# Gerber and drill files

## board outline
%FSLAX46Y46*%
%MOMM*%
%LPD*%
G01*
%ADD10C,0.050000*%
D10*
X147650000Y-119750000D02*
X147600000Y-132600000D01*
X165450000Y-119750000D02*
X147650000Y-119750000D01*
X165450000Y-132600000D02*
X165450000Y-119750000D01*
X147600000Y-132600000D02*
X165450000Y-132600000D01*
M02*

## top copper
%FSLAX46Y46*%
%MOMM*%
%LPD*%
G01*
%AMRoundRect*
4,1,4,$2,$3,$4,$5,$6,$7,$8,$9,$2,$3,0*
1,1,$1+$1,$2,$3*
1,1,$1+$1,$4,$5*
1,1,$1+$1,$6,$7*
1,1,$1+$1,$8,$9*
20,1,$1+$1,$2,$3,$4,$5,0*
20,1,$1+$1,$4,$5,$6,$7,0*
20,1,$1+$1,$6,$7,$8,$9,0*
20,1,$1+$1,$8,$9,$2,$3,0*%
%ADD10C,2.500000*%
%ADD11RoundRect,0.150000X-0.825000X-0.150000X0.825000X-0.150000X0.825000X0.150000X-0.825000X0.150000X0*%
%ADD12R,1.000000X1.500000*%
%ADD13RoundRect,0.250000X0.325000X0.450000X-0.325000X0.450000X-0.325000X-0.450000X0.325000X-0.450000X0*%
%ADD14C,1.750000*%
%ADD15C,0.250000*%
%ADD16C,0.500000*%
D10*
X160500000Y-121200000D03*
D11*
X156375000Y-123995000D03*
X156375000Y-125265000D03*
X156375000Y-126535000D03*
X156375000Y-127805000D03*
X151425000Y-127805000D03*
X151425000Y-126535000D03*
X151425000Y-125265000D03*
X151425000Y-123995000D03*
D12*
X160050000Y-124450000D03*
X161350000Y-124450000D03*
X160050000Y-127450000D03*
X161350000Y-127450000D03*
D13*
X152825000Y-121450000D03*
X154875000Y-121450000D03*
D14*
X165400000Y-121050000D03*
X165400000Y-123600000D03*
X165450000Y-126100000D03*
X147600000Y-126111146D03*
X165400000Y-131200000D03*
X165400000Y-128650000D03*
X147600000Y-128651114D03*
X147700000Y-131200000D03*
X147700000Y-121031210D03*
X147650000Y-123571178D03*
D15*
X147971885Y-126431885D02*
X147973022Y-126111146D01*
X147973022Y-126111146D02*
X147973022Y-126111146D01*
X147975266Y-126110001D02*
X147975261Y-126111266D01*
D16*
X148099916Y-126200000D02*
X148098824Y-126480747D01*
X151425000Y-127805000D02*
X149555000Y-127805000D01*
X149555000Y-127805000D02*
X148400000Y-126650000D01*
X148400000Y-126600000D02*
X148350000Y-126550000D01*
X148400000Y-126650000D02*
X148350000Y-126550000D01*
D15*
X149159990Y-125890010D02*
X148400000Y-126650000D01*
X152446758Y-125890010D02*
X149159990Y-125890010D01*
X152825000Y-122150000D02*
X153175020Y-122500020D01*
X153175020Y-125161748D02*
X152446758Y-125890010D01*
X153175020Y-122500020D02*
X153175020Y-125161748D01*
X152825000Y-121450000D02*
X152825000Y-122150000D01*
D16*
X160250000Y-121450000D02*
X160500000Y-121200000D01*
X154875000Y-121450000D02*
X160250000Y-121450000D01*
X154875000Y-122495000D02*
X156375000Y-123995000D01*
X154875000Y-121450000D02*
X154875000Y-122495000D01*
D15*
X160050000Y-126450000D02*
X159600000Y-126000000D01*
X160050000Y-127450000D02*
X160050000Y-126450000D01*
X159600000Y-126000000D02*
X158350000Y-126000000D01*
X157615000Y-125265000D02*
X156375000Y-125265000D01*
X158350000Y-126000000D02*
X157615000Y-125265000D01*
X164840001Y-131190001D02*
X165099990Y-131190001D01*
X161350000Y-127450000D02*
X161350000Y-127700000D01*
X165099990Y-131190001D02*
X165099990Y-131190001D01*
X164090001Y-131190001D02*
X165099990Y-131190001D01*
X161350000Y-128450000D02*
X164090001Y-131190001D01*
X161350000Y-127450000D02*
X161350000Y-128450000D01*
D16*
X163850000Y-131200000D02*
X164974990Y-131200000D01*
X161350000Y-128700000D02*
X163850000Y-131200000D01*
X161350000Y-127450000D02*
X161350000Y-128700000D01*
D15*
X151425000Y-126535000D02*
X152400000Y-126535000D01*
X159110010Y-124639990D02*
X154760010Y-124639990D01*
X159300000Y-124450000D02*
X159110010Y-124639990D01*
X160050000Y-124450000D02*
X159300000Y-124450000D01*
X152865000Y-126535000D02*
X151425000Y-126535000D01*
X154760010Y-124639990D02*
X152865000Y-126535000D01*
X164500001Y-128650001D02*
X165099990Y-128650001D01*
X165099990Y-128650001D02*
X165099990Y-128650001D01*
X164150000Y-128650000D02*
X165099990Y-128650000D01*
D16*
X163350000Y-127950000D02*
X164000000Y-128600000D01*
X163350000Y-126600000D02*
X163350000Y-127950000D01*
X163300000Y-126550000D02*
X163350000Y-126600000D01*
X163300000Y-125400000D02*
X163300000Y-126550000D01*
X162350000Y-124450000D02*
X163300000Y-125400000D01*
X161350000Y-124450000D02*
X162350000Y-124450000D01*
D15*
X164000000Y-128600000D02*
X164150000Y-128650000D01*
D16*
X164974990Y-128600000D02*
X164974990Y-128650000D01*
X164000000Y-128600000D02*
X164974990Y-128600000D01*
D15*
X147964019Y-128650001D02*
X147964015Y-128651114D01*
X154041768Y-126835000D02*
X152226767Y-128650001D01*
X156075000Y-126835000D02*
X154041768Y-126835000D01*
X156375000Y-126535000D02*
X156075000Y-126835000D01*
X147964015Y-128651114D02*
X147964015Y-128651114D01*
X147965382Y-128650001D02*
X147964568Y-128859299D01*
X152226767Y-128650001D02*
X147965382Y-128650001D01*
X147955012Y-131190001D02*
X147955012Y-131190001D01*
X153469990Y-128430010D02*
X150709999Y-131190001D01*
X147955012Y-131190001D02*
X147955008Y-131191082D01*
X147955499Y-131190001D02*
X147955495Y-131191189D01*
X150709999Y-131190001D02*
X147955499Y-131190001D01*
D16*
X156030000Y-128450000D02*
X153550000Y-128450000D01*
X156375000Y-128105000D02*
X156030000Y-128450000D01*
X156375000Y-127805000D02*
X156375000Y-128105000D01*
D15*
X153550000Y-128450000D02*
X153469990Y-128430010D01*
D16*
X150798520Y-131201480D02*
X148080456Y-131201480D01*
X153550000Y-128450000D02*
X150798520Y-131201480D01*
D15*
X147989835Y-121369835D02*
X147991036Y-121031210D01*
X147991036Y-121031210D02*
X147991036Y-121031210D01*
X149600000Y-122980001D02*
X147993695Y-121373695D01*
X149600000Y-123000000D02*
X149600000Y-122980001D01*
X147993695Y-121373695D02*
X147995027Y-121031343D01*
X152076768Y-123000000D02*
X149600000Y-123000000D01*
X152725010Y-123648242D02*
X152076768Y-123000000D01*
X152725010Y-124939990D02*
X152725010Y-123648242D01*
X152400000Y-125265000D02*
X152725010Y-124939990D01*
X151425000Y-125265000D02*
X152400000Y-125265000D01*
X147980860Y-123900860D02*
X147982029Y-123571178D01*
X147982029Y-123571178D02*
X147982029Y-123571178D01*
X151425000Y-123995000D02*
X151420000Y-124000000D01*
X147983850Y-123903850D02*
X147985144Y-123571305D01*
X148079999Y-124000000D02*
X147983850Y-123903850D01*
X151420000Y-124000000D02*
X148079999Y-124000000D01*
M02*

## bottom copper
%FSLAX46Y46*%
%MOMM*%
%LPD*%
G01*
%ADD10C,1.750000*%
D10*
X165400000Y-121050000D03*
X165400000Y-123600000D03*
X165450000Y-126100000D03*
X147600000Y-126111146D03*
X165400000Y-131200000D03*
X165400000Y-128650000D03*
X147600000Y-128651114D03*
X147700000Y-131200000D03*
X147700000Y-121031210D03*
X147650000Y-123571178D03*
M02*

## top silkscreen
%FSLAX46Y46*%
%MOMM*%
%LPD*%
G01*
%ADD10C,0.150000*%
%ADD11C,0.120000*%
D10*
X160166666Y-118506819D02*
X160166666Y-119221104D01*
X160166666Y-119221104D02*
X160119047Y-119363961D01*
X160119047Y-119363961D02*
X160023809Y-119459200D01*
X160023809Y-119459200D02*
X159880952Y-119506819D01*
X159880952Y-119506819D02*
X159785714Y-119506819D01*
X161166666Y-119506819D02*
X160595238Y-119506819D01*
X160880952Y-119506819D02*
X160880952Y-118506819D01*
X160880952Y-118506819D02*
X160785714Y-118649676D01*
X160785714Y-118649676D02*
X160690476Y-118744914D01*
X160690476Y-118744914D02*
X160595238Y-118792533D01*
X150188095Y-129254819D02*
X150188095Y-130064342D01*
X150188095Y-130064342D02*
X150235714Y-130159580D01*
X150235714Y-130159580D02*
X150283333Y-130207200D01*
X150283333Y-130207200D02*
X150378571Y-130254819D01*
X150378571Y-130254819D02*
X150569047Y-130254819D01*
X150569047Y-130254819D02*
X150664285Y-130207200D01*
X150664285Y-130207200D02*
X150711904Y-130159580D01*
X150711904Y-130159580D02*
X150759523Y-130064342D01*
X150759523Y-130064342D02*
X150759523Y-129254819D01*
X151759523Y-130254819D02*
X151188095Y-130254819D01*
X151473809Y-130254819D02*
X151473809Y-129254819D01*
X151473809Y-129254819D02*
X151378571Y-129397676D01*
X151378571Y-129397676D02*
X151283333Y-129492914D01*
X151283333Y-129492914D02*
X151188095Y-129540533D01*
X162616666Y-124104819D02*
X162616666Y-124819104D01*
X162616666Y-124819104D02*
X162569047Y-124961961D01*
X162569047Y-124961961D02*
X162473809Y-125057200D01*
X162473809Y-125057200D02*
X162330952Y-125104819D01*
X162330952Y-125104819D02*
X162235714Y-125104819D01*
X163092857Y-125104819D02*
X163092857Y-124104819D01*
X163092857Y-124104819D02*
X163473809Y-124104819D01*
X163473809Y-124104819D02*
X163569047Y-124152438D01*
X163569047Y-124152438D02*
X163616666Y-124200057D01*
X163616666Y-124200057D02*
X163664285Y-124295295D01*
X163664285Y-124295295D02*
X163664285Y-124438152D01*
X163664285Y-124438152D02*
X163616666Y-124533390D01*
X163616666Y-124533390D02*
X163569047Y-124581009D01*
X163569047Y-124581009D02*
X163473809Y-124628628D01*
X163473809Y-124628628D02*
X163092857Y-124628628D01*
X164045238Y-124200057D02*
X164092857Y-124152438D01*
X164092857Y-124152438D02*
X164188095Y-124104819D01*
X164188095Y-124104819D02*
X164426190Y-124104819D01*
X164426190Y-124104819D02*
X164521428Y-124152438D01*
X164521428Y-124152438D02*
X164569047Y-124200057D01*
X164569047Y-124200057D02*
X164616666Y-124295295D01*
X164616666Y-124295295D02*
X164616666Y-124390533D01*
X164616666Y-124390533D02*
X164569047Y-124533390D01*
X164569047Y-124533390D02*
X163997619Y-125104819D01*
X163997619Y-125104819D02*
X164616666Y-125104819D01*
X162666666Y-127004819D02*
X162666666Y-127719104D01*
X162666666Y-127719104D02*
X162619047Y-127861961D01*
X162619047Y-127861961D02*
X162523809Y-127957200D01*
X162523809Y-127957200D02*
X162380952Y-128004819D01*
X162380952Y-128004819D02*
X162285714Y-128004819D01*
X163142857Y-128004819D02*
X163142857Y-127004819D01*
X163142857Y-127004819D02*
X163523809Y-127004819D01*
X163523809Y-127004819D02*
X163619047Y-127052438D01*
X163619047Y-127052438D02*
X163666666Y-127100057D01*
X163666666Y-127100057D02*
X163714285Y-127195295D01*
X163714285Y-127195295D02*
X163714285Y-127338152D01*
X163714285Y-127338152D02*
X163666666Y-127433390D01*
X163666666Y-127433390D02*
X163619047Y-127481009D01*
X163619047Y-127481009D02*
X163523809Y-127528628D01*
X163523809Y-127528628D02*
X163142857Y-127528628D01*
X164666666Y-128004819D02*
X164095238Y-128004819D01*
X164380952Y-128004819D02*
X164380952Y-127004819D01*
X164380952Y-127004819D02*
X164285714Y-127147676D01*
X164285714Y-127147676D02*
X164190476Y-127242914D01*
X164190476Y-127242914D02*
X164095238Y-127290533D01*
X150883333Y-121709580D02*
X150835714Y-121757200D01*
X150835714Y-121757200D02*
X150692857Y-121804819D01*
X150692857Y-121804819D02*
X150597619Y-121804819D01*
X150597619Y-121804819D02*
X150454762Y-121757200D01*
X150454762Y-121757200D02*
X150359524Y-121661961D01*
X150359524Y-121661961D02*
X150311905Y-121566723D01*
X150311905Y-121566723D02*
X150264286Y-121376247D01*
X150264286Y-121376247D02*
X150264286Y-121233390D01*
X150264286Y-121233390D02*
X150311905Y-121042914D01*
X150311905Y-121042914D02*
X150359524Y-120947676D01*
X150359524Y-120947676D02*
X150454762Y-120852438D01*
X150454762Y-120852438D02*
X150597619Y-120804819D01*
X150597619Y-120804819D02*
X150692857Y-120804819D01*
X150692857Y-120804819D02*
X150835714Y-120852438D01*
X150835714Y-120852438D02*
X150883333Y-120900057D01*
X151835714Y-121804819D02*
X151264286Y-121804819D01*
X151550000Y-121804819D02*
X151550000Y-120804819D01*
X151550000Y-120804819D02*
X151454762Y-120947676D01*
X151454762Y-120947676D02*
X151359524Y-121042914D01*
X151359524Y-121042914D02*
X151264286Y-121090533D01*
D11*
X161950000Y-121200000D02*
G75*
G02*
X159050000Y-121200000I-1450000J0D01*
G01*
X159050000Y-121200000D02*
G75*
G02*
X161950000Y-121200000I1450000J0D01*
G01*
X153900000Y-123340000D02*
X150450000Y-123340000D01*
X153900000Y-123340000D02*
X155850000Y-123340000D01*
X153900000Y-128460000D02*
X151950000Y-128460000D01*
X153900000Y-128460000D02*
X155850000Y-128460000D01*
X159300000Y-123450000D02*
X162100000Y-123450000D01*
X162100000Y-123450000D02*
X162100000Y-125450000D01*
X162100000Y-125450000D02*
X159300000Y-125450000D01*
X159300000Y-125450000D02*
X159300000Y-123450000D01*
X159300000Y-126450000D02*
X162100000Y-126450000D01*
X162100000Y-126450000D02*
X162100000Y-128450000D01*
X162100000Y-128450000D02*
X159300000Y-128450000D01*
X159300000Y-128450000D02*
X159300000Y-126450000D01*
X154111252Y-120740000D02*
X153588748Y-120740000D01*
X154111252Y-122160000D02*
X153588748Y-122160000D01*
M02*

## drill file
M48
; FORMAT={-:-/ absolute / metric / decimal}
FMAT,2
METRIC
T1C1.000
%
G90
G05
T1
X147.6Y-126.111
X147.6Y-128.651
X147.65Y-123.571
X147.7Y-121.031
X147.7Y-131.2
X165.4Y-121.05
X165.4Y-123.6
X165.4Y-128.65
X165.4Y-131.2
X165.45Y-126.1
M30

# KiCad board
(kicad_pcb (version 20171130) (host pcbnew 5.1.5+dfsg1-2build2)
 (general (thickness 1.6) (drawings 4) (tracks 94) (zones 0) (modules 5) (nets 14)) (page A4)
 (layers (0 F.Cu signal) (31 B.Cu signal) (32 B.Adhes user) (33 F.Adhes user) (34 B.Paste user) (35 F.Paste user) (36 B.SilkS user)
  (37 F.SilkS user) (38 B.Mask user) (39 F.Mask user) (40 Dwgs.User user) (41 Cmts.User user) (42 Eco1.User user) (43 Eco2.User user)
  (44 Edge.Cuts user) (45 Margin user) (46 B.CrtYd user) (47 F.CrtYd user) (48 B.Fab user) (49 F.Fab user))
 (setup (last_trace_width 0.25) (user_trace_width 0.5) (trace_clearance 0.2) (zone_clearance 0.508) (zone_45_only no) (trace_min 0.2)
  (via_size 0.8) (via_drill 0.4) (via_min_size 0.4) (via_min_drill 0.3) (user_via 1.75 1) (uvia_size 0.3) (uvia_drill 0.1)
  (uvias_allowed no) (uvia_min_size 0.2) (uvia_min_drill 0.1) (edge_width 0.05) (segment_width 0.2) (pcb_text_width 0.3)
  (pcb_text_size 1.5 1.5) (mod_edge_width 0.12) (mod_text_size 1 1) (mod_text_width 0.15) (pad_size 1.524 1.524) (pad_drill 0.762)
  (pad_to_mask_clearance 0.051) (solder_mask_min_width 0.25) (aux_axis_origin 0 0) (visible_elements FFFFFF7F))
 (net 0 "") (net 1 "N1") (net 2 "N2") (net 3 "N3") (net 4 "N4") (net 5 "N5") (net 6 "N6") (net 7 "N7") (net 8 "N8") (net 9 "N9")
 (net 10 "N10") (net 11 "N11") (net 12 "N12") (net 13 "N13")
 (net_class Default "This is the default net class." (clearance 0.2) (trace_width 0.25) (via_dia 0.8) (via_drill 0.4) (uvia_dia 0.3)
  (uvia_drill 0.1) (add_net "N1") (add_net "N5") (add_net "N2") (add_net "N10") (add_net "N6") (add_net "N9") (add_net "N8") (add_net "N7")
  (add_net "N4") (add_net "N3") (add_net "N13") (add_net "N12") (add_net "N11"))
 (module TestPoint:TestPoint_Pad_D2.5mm (layer F.Cu) (at 160.5 121.2)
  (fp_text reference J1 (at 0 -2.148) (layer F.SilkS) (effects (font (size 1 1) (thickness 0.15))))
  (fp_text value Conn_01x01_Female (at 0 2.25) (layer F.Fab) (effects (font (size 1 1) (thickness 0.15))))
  (fp_circle (center 0 0) (end 0 1.45) (layer F.SilkS) (width 0.12))
  (pad 1 smd circle (at 0 0) (size 2.5 2.5) (layers F.Cu F.Mask) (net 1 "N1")))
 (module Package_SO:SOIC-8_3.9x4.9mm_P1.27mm (layer F.Cu) (at 153.9 125.9)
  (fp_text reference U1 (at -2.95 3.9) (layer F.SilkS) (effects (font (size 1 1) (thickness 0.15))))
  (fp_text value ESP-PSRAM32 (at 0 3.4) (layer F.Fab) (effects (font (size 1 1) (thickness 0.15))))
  (fp_line (start 0 -2.56) (end -3.45 -2.56) (layer F.SilkS) (width 0.12))
  (fp_line (start 0 -2.56) (end 1.95 -2.56) (layer F.SilkS) (width 0.12))
  (fp_line (start 0 2.56) (end -1.95 2.56) (layer F.SilkS) (width 0.12))
  (fp_line (start 0 2.56) (end 1.95 2.56) (layer F.SilkS) (width 0.12))
  (pad 8 smd roundrect (at 2.475 -1.905) (size 1.95 0.6) (layers F.Cu F.Paste F.Mask) (roundrect_rratio 0.25) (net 1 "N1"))
  (pad 7 smd roundrect (at 2.475 -0.635) (size 1.95 0.6) (layers F.Cu F.Paste F.Mask) (roundrect_rratio 0.25) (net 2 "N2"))
  (pad 6 smd roundrect (at 2.475 0.635) (size 1.95 0.6) (layers F.Cu F.Paste F.Mask) (roundrect_rratio 0.25) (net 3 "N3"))
  (pad 5 smd roundrect (at 2.475 1.905) (size 1.95 0.6) (layers F.Cu F.Paste F.Mask) (roundrect_rratio 0.25) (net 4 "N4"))
  (pad 4 smd roundrect (at -2.475 1.905) (size 1.95 0.6) (layers F.Cu F.Paste F.Mask) (roundrect_rratio 0.25) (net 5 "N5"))
  (pad 3 smd roundrect (at -2.475 0.635) (size 1.95 0.6) (layers F.Cu F.Paste F.Mask) (roundrect_rratio 0.25) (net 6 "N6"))
  (pad 2 smd roundrect (at -2.475 -0.635) (size 1.95 0.6) (layers F.Cu F.Paste F.Mask) (roundrect_rratio 0.25) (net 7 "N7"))
  (pad 1 smd roundrect (at -2.475 -1.905) (size 1.95 0.6) (layers F.Cu F.Paste F.Mask) (roundrect_rratio 0.25) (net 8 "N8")))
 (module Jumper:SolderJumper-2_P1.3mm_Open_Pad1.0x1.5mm (layer F.Cu) (at 160.7 124.45)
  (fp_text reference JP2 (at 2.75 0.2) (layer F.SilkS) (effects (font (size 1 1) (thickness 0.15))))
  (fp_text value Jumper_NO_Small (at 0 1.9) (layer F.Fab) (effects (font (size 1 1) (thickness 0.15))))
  (fp_line (start -1.4 -1) (end 1.4 -1) (layer F.SilkS) (width 0.12))
  (fp_line (start 1.4 -1) (end 1.4 1) (layer F.SilkS) (width 0.12))
  (fp_line (start 1.4 1) (end -1.4 1) (layer F.SilkS) (width 0.12))
  (fp_line (start -1.4 1) (end -1.4 -1) (layer F.SilkS) (width 0.12))
  (pad 1 smd rect (at -0.65 0) (size 1 1.5) (layers F.Cu F.Mask) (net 6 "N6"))
  (pad 2 smd rect (at 0.65 0) (size 1 1.5) (layers F.Cu F.Mask) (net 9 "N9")))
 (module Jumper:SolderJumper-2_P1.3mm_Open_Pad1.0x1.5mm (layer F.Cu) (at 160.7 127.45)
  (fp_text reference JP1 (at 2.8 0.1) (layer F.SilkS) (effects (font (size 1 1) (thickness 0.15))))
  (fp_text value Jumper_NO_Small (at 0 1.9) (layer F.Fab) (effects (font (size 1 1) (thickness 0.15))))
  (fp_line (start -1.4 -1) (end 1.4 -1) (layer F.SilkS) (width 0.12))
  (fp_line (start 1.4 -1) (end 1.4 1) (layer F.SilkS) (width 0.12))
  (fp_line (start 1.4 1) (end -1.4 1) (layer F.SilkS) (width 0.12))
  (fp_line (start -1.4 1) (end -1.4 -1) (layer F.SilkS) (width 0.12))
  (pad 1 smd rect (at -0.65 0) (size 1 1.5) (layers F.Cu F.Mask) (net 2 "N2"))
  (pad 2 smd rect (at 0.65 0) (size 1 1.5) (layers F.Cu F.Mask) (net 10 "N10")))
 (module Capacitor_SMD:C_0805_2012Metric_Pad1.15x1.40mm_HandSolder (layer F.Cu) (at 153.85 121.45 180)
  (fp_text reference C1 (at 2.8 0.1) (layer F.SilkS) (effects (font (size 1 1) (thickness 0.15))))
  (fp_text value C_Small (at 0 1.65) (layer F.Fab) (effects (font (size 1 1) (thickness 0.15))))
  (fp_line (start -0.261252 0.71) (end 0.261252 0.71) (layer F.SilkS) (width 0.12))
  (fp_line (start -0.261252 -0.71) (end 0.261252 -0.71) (layer F.SilkS) (width 0.12))
  (pad 2 smd roundrect (at 1.025 0 180) (size 1.15 1.4) (layers F.Cu F.Paste F.Mask) (roundrect_rratio 0.217391) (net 5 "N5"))
  (pad 1 smd roundrect (at -1.025 0 180) (size 1.15 1.4) (layers F.Cu F.Paste F.Mask) (roundrect_rratio 0.217391) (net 1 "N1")))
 (gr_line (start 147.65 119.75) (end 147.6 132.6) (layer Edge.Cuts) (width 0.05))
 (gr_line (start 165.45 119.75) (end 147.65 119.75) (layer Edge.Cuts) (width 0.05))
 (gr_line (start 165.45 132.6) (end 165.45 119.75) (layer Edge.Cuts) (width 0.05))
 (gr_line (start 147.6 132.6) (end 165.45 132.6) (layer Edge.Cuts) (width 0.05))
 (via (at 165.4 121.05) (size 1.75) (drill 1) (layers F.Cu B.Cu) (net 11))
 (via (at 165.4 123.6) (size 1.75) (drill 1) (layers F.Cu B.Cu) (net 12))
 (via (at 165.45 126.1) (size 1.75) (drill 1) (layers F.Cu B.Cu) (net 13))
 (segment (start 147.971885 126.431885) (end 147.973022 126.111146) (width 0.25) (layer F.Cu) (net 5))
 (segment (start 147.973022 126.111146) (end 147.973022 126.111146) (width 0.25) (layer F.Cu) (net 5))
 (via (at 147.6 126.111146) (size 1.75) (drill 1) (layers F.Cu B.Cu) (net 5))
 (segment (start 147.975266 126.110001) (end 147.975261 126.111266) (width 0.25) (layer F.Cu) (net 5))
 (segment (start 148.099916 126.2) (end 148.098824 126.480747) (width 0.5) (layer F.Cu) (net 5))
 (segment (start 151.425 127.805) (end 149.555 127.805) (width 0.5) (layer F.Cu) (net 5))
 (segment (start 149.555 127.805) (end 148.4 126.65) (width 0.5) (layer F.Cu) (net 5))
 (segment (start 148.4 126.6) (end 148.35 126.55) (width 0.5) (layer F.Cu) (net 5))
 (segment (start 148.4 126.65) (end 148.35 126.55) (width 0.5) (layer F.Cu) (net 5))
 (segment (start 149.15999 125.89001) (end 148.4 126.65) (width 0.25) (layer F.Cu) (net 5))
 (segment (start 152.446758 125.89001) (end 149.15999 125.89001) (width 0.25) (layer F.Cu) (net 5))
 (segment (start 152.825 122.15) (end 153.17502 122.50002) (width 0.25) (layer F.Cu) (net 5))
 (segment (start 153.17502 125.161748) (end 152.446758 125.89001) (width 0.25) (layer F.Cu) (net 5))
 (segment (start 153.17502 122.50002) (end 153.17502 125.161748) (width 0.25) (layer F.Cu) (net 5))
 (segment (start 152.825 121.45) (end 152.825 122.15) (width 0.25) (layer F.Cu) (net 5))
 (segment (start 160.25 121.45) (end 160.5 121.2) (width 0.5) (layer F.Cu) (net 1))
 (segment (start 154.875 121.45) (end 160.25 121.45) (width 0.5) (layer F.Cu) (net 1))
 (segment (start 154.875 122.495) (end 156.375 123.995) (width 0.5) (layer F.Cu) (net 1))
 (segment (start 154.875 121.45) (end 154.875 122.495) (width 0.5) (layer F.Cu) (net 1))
 (segment (start 160.05 126.45) (end 159.6 126) (width 0.25) (layer F.Cu) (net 2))
 (segment (start 160.05 127.45) (end 160.05 126.45) (width 0.25) (layer F.Cu) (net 2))
 (segment (start 159.6 126) (end 158.35 126) (width 0.25) (layer F.Cu) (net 2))
 (segment (start 157.615 125.265) (end 156.375 125.265) (width 0.25) (layer F.Cu) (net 2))
 (segment (start 158.35 126) (end 157.615 125.265) (width 0.25) (layer F.Cu) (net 2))
 (segment (start 164.840001 131.190001) (end 165.09999 131.190001) (width 0.25) (layer F.Cu) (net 10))
 (segment (start 161.35 127.45) (end 161.35 127.7) (width 0.25) (layer F.Cu) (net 10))
 (segment (start 165.09999 131.190001) (end 165.09999 131.190001) (width 0.25) (layer F.Cu) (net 10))
 (via (at 165.4 131.2) (size 1.75) (drill 1) (layers F.Cu B.Cu) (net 10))
 (segment (start 164.090001 131.190001) (end 165.09999 131.190001) (width 0.25) (layer F.Cu) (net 10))
 (segment (start 161.35 128.45) (end 164.090001 131.190001) (width 0.25) (layer F.Cu) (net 10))
 (segment (start 161.35 127.45) (end 161.35 128.45) (width 0.25) (layer F.Cu) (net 10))
 (segment (start 163.85 131.2) (end 164.97499 131.2) (width 0.5) (layer F.Cu) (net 10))
 (segment (start 161.35 128.7) (end 163.85 131.2) (width 0.5) (layer F.Cu) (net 10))
 (segment (start 161.35 127.45) (end 161.35 128.7) (width 0.5) (layer F.Cu) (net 10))
 (segment (start 151.425 126.535) (end 152.4 126.535) (width 0.25) (layer F.Cu) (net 6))
 (segment (start 159.11001 124.63999) (end 154.76001 124.63999) (width 0.25) (layer F.Cu) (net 6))
 (segment (start 159.3 124.45) (end 159.11001 124.63999) (width 0.25) (layer F.Cu) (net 6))
 (segment (start 160.05 124.45) (end 159.3 124.45) (width 0.25) (layer F.Cu) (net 6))
 (segment (start 152.865 126.535) (end 151.425 126.535) (width 0.25) (layer F.Cu) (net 6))
 (segment (start 154.76001 124.63999) (end 152.865 126.535) (width 0.25) (layer F.Cu) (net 6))
 (segment (start 164.500001 128.650001) (end 165.09999 128.650001) (width 0.25) (layer F.Cu) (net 9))
 (segment (start 165.09999 128.650001) (end 165.09999 128.650001) (width 0.25) (layer F.Cu) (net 9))
 (via (at 165.4 128.65) (size 1.75) (drill 1) (layers F.Cu B.Cu) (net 9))
 (segment (start 164.15 128.65) (end 165.09999 128.65) (width 0.25) (layer F.Cu) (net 9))
 (segment (start 163.35 127.95) (end 164 128.6) (width 0.5) (layer F.Cu) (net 9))
 (segment (start 163.35 126.6) (end 163.35 127.95) (width 0.5) (layer F.Cu) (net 9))
 (segment (start 163.3 126.55) (end 163.35 126.6) (width 0.5) (layer F.Cu) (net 9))
 (segment (start 163.3 125.4) (end 163.3 126.55) (width 0.5) (layer F.Cu) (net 9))
 (segment (start 162.35 124.45) (end 163.3 125.4) (width 0.5) (layer F.Cu) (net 9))
 (segment (start 161.35 124.45) (end 162.35 124.45) (width 0.5) (layer F.Cu) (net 9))
 (segment (start 164 128.6) (end 164.15 128.65) (width 0.25) (layer F.Cu) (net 9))
 (segment (start 164.97499 128.6) (end 164.97499 128.65) (width 0.5) (layer F.Cu) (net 9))
 (segment (start 164 128.6) (end 164.97499 128.6) (width 0.5) (layer F.Cu) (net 9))
 (segment (start 147.964019 128.650001) (end 147.964015 128.651114) (width 0.25) (layer F.Cu) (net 3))
 (segment (start 154.041768 126.835) (end 152.226767 128.650001) (width 0.25) (layer F.Cu) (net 3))
 (segment (start 156.075 126.835) (end 154.041768 126.835) (width 0.25) (layer F.Cu) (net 3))
 (segment (start 156.375 126.535) (end 156.075 126.835) (width 0.25) (layer F.Cu) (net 3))
 (segment (start 147.964015 128.651114) (end 147.964015 128.651114) (width 0.25) (layer F.Cu) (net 3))
 (via (at 147.6 128.651114) (size 1.75) (drill 1) (layers F.Cu B.Cu) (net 3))
 (segment (start 147.965382 128.650001) (end 147.964568 128.859299) (width 0.25) (layer F.Cu) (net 3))
 (segment (start 152.226767 128.650001) (end 147.965382 128.650001) (width 0.25) (layer F.Cu) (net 3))
 (segment (start 147.955012 131.190001) (end 147.955012 131.190001) (width 0.25) (layer F.Cu) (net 4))
 (segment (start 153.46999 128.43001) (end 150.709999 131.190001) (width 0.25) (layer F.Cu) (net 4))
 (segment (start 147.955012 131.190001) (end 147.955008 131.191082) (width 0.25) (layer F.Cu) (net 4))
 (via (at 147.7 131.2) (size 1.75) (drill 1) (layers F.Cu B.Cu) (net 4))
 (segment (start 147.955499 131.190001) (end 147.955495 131.191189) (width 0.25) (layer F.Cu) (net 4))
 (segment (start 150.709999 131.190001) (end 147.955499 131.190001) (width 0.25) (layer F.Cu) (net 4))
 (segment (start 156.03 128.45) (end 153.55 128.45) (width 0.5) (layer F.Cu) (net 4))
 (segment (start 156.375 128.105) (end 156.03 128.45) (width 0.5) (layer F.Cu) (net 4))
 (segment (start 156.375 127.805) (end 156.375 128.105) (width 0.5) (layer F.Cu) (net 4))
 (segment (start 153.55 128.45) (end 153.46999 128.43001) (width 0.25) (layer F.Cu) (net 4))
 (segment (start 150.79852 131.20148) (end 148.080456 131.20148) (width 0.5) (layer F.Cu) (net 4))
 (segment (start 153.55 128.45) (end 150.79852 131.20148) (width 0.5) (layer F.Cu) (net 4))
 (segment (start 147.989835 121.369835) (end 147.991036 121.03121) (width 0.25) (layer F.Cu) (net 7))
 (segment (start 147.991036 121.03121) (end 147.991036 121.03121) (width 0.25) (layer F.Cu) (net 7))
 (via (at 147.7 121.03121) (size 1.75) (drill 1) (layers F.Cu B.Cu) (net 7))
 (segment (start 149.6 122.980001) (end 147.993695 121.373695) (width 0.25) (layer F.Cu) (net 7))
 (segment (start 149.6 123) (end 149.6 122.980001) (width 0.25) (layer F.Cu) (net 7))
 (segment (start 147.993695 121.373695) (end 147.995027 121.031343) (width 0.25) (layer F.Cu) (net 7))
 (segment (start 152.076768 123) (end 149.6 123) (width 0.25) (layer F.Cu) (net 7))
 (segment (start 152.72501 123.648242) (end 152.076768 123) (width 0.25) (layer F.Cu) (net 7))
 (segment (start 152.72501 124.93999) (end 152.72501 123.648242) (width 0.25) (layer F.Cu) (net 7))
 (segment (start 152.4 125.265) (end 152.72501 124.93999) (width 0.25) (layer F.Cu) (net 7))
 (segment (start 151.425 125.265) (end 152.4 125.265) (width 0.25) (layer F.Cu) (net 7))
 (segment (start 147.98086 123.90086) (end 147.982029 123.571178) (width 0.25) (layer F.Cu) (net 8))
 (segment (start 147.982029 123.571178) (end 147.982029 123.571178) (width 0.25) (layer F.Cu) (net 8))
 (via (at 147.65 123.571178) (size 1.75) (drill 1) (layers F.Cu B.Cu) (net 8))
 (segment (start 151.425 123.995) (end 151.42 124) (width 0.25) (layer F.Cu) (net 8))
 (segment (start 147.98385 123.90385) (end 147.985144 123.571305) (width 0.25) (layer F.Cu) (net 8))
 (segment (start 148.079999 124) (end 147.98385 123.90385) (width 0.25) (layer F.Cu) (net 8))
 (segment (start 151.42 124) (end 148.079999 124) (width 0.25) (layer F.Cu) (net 8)))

